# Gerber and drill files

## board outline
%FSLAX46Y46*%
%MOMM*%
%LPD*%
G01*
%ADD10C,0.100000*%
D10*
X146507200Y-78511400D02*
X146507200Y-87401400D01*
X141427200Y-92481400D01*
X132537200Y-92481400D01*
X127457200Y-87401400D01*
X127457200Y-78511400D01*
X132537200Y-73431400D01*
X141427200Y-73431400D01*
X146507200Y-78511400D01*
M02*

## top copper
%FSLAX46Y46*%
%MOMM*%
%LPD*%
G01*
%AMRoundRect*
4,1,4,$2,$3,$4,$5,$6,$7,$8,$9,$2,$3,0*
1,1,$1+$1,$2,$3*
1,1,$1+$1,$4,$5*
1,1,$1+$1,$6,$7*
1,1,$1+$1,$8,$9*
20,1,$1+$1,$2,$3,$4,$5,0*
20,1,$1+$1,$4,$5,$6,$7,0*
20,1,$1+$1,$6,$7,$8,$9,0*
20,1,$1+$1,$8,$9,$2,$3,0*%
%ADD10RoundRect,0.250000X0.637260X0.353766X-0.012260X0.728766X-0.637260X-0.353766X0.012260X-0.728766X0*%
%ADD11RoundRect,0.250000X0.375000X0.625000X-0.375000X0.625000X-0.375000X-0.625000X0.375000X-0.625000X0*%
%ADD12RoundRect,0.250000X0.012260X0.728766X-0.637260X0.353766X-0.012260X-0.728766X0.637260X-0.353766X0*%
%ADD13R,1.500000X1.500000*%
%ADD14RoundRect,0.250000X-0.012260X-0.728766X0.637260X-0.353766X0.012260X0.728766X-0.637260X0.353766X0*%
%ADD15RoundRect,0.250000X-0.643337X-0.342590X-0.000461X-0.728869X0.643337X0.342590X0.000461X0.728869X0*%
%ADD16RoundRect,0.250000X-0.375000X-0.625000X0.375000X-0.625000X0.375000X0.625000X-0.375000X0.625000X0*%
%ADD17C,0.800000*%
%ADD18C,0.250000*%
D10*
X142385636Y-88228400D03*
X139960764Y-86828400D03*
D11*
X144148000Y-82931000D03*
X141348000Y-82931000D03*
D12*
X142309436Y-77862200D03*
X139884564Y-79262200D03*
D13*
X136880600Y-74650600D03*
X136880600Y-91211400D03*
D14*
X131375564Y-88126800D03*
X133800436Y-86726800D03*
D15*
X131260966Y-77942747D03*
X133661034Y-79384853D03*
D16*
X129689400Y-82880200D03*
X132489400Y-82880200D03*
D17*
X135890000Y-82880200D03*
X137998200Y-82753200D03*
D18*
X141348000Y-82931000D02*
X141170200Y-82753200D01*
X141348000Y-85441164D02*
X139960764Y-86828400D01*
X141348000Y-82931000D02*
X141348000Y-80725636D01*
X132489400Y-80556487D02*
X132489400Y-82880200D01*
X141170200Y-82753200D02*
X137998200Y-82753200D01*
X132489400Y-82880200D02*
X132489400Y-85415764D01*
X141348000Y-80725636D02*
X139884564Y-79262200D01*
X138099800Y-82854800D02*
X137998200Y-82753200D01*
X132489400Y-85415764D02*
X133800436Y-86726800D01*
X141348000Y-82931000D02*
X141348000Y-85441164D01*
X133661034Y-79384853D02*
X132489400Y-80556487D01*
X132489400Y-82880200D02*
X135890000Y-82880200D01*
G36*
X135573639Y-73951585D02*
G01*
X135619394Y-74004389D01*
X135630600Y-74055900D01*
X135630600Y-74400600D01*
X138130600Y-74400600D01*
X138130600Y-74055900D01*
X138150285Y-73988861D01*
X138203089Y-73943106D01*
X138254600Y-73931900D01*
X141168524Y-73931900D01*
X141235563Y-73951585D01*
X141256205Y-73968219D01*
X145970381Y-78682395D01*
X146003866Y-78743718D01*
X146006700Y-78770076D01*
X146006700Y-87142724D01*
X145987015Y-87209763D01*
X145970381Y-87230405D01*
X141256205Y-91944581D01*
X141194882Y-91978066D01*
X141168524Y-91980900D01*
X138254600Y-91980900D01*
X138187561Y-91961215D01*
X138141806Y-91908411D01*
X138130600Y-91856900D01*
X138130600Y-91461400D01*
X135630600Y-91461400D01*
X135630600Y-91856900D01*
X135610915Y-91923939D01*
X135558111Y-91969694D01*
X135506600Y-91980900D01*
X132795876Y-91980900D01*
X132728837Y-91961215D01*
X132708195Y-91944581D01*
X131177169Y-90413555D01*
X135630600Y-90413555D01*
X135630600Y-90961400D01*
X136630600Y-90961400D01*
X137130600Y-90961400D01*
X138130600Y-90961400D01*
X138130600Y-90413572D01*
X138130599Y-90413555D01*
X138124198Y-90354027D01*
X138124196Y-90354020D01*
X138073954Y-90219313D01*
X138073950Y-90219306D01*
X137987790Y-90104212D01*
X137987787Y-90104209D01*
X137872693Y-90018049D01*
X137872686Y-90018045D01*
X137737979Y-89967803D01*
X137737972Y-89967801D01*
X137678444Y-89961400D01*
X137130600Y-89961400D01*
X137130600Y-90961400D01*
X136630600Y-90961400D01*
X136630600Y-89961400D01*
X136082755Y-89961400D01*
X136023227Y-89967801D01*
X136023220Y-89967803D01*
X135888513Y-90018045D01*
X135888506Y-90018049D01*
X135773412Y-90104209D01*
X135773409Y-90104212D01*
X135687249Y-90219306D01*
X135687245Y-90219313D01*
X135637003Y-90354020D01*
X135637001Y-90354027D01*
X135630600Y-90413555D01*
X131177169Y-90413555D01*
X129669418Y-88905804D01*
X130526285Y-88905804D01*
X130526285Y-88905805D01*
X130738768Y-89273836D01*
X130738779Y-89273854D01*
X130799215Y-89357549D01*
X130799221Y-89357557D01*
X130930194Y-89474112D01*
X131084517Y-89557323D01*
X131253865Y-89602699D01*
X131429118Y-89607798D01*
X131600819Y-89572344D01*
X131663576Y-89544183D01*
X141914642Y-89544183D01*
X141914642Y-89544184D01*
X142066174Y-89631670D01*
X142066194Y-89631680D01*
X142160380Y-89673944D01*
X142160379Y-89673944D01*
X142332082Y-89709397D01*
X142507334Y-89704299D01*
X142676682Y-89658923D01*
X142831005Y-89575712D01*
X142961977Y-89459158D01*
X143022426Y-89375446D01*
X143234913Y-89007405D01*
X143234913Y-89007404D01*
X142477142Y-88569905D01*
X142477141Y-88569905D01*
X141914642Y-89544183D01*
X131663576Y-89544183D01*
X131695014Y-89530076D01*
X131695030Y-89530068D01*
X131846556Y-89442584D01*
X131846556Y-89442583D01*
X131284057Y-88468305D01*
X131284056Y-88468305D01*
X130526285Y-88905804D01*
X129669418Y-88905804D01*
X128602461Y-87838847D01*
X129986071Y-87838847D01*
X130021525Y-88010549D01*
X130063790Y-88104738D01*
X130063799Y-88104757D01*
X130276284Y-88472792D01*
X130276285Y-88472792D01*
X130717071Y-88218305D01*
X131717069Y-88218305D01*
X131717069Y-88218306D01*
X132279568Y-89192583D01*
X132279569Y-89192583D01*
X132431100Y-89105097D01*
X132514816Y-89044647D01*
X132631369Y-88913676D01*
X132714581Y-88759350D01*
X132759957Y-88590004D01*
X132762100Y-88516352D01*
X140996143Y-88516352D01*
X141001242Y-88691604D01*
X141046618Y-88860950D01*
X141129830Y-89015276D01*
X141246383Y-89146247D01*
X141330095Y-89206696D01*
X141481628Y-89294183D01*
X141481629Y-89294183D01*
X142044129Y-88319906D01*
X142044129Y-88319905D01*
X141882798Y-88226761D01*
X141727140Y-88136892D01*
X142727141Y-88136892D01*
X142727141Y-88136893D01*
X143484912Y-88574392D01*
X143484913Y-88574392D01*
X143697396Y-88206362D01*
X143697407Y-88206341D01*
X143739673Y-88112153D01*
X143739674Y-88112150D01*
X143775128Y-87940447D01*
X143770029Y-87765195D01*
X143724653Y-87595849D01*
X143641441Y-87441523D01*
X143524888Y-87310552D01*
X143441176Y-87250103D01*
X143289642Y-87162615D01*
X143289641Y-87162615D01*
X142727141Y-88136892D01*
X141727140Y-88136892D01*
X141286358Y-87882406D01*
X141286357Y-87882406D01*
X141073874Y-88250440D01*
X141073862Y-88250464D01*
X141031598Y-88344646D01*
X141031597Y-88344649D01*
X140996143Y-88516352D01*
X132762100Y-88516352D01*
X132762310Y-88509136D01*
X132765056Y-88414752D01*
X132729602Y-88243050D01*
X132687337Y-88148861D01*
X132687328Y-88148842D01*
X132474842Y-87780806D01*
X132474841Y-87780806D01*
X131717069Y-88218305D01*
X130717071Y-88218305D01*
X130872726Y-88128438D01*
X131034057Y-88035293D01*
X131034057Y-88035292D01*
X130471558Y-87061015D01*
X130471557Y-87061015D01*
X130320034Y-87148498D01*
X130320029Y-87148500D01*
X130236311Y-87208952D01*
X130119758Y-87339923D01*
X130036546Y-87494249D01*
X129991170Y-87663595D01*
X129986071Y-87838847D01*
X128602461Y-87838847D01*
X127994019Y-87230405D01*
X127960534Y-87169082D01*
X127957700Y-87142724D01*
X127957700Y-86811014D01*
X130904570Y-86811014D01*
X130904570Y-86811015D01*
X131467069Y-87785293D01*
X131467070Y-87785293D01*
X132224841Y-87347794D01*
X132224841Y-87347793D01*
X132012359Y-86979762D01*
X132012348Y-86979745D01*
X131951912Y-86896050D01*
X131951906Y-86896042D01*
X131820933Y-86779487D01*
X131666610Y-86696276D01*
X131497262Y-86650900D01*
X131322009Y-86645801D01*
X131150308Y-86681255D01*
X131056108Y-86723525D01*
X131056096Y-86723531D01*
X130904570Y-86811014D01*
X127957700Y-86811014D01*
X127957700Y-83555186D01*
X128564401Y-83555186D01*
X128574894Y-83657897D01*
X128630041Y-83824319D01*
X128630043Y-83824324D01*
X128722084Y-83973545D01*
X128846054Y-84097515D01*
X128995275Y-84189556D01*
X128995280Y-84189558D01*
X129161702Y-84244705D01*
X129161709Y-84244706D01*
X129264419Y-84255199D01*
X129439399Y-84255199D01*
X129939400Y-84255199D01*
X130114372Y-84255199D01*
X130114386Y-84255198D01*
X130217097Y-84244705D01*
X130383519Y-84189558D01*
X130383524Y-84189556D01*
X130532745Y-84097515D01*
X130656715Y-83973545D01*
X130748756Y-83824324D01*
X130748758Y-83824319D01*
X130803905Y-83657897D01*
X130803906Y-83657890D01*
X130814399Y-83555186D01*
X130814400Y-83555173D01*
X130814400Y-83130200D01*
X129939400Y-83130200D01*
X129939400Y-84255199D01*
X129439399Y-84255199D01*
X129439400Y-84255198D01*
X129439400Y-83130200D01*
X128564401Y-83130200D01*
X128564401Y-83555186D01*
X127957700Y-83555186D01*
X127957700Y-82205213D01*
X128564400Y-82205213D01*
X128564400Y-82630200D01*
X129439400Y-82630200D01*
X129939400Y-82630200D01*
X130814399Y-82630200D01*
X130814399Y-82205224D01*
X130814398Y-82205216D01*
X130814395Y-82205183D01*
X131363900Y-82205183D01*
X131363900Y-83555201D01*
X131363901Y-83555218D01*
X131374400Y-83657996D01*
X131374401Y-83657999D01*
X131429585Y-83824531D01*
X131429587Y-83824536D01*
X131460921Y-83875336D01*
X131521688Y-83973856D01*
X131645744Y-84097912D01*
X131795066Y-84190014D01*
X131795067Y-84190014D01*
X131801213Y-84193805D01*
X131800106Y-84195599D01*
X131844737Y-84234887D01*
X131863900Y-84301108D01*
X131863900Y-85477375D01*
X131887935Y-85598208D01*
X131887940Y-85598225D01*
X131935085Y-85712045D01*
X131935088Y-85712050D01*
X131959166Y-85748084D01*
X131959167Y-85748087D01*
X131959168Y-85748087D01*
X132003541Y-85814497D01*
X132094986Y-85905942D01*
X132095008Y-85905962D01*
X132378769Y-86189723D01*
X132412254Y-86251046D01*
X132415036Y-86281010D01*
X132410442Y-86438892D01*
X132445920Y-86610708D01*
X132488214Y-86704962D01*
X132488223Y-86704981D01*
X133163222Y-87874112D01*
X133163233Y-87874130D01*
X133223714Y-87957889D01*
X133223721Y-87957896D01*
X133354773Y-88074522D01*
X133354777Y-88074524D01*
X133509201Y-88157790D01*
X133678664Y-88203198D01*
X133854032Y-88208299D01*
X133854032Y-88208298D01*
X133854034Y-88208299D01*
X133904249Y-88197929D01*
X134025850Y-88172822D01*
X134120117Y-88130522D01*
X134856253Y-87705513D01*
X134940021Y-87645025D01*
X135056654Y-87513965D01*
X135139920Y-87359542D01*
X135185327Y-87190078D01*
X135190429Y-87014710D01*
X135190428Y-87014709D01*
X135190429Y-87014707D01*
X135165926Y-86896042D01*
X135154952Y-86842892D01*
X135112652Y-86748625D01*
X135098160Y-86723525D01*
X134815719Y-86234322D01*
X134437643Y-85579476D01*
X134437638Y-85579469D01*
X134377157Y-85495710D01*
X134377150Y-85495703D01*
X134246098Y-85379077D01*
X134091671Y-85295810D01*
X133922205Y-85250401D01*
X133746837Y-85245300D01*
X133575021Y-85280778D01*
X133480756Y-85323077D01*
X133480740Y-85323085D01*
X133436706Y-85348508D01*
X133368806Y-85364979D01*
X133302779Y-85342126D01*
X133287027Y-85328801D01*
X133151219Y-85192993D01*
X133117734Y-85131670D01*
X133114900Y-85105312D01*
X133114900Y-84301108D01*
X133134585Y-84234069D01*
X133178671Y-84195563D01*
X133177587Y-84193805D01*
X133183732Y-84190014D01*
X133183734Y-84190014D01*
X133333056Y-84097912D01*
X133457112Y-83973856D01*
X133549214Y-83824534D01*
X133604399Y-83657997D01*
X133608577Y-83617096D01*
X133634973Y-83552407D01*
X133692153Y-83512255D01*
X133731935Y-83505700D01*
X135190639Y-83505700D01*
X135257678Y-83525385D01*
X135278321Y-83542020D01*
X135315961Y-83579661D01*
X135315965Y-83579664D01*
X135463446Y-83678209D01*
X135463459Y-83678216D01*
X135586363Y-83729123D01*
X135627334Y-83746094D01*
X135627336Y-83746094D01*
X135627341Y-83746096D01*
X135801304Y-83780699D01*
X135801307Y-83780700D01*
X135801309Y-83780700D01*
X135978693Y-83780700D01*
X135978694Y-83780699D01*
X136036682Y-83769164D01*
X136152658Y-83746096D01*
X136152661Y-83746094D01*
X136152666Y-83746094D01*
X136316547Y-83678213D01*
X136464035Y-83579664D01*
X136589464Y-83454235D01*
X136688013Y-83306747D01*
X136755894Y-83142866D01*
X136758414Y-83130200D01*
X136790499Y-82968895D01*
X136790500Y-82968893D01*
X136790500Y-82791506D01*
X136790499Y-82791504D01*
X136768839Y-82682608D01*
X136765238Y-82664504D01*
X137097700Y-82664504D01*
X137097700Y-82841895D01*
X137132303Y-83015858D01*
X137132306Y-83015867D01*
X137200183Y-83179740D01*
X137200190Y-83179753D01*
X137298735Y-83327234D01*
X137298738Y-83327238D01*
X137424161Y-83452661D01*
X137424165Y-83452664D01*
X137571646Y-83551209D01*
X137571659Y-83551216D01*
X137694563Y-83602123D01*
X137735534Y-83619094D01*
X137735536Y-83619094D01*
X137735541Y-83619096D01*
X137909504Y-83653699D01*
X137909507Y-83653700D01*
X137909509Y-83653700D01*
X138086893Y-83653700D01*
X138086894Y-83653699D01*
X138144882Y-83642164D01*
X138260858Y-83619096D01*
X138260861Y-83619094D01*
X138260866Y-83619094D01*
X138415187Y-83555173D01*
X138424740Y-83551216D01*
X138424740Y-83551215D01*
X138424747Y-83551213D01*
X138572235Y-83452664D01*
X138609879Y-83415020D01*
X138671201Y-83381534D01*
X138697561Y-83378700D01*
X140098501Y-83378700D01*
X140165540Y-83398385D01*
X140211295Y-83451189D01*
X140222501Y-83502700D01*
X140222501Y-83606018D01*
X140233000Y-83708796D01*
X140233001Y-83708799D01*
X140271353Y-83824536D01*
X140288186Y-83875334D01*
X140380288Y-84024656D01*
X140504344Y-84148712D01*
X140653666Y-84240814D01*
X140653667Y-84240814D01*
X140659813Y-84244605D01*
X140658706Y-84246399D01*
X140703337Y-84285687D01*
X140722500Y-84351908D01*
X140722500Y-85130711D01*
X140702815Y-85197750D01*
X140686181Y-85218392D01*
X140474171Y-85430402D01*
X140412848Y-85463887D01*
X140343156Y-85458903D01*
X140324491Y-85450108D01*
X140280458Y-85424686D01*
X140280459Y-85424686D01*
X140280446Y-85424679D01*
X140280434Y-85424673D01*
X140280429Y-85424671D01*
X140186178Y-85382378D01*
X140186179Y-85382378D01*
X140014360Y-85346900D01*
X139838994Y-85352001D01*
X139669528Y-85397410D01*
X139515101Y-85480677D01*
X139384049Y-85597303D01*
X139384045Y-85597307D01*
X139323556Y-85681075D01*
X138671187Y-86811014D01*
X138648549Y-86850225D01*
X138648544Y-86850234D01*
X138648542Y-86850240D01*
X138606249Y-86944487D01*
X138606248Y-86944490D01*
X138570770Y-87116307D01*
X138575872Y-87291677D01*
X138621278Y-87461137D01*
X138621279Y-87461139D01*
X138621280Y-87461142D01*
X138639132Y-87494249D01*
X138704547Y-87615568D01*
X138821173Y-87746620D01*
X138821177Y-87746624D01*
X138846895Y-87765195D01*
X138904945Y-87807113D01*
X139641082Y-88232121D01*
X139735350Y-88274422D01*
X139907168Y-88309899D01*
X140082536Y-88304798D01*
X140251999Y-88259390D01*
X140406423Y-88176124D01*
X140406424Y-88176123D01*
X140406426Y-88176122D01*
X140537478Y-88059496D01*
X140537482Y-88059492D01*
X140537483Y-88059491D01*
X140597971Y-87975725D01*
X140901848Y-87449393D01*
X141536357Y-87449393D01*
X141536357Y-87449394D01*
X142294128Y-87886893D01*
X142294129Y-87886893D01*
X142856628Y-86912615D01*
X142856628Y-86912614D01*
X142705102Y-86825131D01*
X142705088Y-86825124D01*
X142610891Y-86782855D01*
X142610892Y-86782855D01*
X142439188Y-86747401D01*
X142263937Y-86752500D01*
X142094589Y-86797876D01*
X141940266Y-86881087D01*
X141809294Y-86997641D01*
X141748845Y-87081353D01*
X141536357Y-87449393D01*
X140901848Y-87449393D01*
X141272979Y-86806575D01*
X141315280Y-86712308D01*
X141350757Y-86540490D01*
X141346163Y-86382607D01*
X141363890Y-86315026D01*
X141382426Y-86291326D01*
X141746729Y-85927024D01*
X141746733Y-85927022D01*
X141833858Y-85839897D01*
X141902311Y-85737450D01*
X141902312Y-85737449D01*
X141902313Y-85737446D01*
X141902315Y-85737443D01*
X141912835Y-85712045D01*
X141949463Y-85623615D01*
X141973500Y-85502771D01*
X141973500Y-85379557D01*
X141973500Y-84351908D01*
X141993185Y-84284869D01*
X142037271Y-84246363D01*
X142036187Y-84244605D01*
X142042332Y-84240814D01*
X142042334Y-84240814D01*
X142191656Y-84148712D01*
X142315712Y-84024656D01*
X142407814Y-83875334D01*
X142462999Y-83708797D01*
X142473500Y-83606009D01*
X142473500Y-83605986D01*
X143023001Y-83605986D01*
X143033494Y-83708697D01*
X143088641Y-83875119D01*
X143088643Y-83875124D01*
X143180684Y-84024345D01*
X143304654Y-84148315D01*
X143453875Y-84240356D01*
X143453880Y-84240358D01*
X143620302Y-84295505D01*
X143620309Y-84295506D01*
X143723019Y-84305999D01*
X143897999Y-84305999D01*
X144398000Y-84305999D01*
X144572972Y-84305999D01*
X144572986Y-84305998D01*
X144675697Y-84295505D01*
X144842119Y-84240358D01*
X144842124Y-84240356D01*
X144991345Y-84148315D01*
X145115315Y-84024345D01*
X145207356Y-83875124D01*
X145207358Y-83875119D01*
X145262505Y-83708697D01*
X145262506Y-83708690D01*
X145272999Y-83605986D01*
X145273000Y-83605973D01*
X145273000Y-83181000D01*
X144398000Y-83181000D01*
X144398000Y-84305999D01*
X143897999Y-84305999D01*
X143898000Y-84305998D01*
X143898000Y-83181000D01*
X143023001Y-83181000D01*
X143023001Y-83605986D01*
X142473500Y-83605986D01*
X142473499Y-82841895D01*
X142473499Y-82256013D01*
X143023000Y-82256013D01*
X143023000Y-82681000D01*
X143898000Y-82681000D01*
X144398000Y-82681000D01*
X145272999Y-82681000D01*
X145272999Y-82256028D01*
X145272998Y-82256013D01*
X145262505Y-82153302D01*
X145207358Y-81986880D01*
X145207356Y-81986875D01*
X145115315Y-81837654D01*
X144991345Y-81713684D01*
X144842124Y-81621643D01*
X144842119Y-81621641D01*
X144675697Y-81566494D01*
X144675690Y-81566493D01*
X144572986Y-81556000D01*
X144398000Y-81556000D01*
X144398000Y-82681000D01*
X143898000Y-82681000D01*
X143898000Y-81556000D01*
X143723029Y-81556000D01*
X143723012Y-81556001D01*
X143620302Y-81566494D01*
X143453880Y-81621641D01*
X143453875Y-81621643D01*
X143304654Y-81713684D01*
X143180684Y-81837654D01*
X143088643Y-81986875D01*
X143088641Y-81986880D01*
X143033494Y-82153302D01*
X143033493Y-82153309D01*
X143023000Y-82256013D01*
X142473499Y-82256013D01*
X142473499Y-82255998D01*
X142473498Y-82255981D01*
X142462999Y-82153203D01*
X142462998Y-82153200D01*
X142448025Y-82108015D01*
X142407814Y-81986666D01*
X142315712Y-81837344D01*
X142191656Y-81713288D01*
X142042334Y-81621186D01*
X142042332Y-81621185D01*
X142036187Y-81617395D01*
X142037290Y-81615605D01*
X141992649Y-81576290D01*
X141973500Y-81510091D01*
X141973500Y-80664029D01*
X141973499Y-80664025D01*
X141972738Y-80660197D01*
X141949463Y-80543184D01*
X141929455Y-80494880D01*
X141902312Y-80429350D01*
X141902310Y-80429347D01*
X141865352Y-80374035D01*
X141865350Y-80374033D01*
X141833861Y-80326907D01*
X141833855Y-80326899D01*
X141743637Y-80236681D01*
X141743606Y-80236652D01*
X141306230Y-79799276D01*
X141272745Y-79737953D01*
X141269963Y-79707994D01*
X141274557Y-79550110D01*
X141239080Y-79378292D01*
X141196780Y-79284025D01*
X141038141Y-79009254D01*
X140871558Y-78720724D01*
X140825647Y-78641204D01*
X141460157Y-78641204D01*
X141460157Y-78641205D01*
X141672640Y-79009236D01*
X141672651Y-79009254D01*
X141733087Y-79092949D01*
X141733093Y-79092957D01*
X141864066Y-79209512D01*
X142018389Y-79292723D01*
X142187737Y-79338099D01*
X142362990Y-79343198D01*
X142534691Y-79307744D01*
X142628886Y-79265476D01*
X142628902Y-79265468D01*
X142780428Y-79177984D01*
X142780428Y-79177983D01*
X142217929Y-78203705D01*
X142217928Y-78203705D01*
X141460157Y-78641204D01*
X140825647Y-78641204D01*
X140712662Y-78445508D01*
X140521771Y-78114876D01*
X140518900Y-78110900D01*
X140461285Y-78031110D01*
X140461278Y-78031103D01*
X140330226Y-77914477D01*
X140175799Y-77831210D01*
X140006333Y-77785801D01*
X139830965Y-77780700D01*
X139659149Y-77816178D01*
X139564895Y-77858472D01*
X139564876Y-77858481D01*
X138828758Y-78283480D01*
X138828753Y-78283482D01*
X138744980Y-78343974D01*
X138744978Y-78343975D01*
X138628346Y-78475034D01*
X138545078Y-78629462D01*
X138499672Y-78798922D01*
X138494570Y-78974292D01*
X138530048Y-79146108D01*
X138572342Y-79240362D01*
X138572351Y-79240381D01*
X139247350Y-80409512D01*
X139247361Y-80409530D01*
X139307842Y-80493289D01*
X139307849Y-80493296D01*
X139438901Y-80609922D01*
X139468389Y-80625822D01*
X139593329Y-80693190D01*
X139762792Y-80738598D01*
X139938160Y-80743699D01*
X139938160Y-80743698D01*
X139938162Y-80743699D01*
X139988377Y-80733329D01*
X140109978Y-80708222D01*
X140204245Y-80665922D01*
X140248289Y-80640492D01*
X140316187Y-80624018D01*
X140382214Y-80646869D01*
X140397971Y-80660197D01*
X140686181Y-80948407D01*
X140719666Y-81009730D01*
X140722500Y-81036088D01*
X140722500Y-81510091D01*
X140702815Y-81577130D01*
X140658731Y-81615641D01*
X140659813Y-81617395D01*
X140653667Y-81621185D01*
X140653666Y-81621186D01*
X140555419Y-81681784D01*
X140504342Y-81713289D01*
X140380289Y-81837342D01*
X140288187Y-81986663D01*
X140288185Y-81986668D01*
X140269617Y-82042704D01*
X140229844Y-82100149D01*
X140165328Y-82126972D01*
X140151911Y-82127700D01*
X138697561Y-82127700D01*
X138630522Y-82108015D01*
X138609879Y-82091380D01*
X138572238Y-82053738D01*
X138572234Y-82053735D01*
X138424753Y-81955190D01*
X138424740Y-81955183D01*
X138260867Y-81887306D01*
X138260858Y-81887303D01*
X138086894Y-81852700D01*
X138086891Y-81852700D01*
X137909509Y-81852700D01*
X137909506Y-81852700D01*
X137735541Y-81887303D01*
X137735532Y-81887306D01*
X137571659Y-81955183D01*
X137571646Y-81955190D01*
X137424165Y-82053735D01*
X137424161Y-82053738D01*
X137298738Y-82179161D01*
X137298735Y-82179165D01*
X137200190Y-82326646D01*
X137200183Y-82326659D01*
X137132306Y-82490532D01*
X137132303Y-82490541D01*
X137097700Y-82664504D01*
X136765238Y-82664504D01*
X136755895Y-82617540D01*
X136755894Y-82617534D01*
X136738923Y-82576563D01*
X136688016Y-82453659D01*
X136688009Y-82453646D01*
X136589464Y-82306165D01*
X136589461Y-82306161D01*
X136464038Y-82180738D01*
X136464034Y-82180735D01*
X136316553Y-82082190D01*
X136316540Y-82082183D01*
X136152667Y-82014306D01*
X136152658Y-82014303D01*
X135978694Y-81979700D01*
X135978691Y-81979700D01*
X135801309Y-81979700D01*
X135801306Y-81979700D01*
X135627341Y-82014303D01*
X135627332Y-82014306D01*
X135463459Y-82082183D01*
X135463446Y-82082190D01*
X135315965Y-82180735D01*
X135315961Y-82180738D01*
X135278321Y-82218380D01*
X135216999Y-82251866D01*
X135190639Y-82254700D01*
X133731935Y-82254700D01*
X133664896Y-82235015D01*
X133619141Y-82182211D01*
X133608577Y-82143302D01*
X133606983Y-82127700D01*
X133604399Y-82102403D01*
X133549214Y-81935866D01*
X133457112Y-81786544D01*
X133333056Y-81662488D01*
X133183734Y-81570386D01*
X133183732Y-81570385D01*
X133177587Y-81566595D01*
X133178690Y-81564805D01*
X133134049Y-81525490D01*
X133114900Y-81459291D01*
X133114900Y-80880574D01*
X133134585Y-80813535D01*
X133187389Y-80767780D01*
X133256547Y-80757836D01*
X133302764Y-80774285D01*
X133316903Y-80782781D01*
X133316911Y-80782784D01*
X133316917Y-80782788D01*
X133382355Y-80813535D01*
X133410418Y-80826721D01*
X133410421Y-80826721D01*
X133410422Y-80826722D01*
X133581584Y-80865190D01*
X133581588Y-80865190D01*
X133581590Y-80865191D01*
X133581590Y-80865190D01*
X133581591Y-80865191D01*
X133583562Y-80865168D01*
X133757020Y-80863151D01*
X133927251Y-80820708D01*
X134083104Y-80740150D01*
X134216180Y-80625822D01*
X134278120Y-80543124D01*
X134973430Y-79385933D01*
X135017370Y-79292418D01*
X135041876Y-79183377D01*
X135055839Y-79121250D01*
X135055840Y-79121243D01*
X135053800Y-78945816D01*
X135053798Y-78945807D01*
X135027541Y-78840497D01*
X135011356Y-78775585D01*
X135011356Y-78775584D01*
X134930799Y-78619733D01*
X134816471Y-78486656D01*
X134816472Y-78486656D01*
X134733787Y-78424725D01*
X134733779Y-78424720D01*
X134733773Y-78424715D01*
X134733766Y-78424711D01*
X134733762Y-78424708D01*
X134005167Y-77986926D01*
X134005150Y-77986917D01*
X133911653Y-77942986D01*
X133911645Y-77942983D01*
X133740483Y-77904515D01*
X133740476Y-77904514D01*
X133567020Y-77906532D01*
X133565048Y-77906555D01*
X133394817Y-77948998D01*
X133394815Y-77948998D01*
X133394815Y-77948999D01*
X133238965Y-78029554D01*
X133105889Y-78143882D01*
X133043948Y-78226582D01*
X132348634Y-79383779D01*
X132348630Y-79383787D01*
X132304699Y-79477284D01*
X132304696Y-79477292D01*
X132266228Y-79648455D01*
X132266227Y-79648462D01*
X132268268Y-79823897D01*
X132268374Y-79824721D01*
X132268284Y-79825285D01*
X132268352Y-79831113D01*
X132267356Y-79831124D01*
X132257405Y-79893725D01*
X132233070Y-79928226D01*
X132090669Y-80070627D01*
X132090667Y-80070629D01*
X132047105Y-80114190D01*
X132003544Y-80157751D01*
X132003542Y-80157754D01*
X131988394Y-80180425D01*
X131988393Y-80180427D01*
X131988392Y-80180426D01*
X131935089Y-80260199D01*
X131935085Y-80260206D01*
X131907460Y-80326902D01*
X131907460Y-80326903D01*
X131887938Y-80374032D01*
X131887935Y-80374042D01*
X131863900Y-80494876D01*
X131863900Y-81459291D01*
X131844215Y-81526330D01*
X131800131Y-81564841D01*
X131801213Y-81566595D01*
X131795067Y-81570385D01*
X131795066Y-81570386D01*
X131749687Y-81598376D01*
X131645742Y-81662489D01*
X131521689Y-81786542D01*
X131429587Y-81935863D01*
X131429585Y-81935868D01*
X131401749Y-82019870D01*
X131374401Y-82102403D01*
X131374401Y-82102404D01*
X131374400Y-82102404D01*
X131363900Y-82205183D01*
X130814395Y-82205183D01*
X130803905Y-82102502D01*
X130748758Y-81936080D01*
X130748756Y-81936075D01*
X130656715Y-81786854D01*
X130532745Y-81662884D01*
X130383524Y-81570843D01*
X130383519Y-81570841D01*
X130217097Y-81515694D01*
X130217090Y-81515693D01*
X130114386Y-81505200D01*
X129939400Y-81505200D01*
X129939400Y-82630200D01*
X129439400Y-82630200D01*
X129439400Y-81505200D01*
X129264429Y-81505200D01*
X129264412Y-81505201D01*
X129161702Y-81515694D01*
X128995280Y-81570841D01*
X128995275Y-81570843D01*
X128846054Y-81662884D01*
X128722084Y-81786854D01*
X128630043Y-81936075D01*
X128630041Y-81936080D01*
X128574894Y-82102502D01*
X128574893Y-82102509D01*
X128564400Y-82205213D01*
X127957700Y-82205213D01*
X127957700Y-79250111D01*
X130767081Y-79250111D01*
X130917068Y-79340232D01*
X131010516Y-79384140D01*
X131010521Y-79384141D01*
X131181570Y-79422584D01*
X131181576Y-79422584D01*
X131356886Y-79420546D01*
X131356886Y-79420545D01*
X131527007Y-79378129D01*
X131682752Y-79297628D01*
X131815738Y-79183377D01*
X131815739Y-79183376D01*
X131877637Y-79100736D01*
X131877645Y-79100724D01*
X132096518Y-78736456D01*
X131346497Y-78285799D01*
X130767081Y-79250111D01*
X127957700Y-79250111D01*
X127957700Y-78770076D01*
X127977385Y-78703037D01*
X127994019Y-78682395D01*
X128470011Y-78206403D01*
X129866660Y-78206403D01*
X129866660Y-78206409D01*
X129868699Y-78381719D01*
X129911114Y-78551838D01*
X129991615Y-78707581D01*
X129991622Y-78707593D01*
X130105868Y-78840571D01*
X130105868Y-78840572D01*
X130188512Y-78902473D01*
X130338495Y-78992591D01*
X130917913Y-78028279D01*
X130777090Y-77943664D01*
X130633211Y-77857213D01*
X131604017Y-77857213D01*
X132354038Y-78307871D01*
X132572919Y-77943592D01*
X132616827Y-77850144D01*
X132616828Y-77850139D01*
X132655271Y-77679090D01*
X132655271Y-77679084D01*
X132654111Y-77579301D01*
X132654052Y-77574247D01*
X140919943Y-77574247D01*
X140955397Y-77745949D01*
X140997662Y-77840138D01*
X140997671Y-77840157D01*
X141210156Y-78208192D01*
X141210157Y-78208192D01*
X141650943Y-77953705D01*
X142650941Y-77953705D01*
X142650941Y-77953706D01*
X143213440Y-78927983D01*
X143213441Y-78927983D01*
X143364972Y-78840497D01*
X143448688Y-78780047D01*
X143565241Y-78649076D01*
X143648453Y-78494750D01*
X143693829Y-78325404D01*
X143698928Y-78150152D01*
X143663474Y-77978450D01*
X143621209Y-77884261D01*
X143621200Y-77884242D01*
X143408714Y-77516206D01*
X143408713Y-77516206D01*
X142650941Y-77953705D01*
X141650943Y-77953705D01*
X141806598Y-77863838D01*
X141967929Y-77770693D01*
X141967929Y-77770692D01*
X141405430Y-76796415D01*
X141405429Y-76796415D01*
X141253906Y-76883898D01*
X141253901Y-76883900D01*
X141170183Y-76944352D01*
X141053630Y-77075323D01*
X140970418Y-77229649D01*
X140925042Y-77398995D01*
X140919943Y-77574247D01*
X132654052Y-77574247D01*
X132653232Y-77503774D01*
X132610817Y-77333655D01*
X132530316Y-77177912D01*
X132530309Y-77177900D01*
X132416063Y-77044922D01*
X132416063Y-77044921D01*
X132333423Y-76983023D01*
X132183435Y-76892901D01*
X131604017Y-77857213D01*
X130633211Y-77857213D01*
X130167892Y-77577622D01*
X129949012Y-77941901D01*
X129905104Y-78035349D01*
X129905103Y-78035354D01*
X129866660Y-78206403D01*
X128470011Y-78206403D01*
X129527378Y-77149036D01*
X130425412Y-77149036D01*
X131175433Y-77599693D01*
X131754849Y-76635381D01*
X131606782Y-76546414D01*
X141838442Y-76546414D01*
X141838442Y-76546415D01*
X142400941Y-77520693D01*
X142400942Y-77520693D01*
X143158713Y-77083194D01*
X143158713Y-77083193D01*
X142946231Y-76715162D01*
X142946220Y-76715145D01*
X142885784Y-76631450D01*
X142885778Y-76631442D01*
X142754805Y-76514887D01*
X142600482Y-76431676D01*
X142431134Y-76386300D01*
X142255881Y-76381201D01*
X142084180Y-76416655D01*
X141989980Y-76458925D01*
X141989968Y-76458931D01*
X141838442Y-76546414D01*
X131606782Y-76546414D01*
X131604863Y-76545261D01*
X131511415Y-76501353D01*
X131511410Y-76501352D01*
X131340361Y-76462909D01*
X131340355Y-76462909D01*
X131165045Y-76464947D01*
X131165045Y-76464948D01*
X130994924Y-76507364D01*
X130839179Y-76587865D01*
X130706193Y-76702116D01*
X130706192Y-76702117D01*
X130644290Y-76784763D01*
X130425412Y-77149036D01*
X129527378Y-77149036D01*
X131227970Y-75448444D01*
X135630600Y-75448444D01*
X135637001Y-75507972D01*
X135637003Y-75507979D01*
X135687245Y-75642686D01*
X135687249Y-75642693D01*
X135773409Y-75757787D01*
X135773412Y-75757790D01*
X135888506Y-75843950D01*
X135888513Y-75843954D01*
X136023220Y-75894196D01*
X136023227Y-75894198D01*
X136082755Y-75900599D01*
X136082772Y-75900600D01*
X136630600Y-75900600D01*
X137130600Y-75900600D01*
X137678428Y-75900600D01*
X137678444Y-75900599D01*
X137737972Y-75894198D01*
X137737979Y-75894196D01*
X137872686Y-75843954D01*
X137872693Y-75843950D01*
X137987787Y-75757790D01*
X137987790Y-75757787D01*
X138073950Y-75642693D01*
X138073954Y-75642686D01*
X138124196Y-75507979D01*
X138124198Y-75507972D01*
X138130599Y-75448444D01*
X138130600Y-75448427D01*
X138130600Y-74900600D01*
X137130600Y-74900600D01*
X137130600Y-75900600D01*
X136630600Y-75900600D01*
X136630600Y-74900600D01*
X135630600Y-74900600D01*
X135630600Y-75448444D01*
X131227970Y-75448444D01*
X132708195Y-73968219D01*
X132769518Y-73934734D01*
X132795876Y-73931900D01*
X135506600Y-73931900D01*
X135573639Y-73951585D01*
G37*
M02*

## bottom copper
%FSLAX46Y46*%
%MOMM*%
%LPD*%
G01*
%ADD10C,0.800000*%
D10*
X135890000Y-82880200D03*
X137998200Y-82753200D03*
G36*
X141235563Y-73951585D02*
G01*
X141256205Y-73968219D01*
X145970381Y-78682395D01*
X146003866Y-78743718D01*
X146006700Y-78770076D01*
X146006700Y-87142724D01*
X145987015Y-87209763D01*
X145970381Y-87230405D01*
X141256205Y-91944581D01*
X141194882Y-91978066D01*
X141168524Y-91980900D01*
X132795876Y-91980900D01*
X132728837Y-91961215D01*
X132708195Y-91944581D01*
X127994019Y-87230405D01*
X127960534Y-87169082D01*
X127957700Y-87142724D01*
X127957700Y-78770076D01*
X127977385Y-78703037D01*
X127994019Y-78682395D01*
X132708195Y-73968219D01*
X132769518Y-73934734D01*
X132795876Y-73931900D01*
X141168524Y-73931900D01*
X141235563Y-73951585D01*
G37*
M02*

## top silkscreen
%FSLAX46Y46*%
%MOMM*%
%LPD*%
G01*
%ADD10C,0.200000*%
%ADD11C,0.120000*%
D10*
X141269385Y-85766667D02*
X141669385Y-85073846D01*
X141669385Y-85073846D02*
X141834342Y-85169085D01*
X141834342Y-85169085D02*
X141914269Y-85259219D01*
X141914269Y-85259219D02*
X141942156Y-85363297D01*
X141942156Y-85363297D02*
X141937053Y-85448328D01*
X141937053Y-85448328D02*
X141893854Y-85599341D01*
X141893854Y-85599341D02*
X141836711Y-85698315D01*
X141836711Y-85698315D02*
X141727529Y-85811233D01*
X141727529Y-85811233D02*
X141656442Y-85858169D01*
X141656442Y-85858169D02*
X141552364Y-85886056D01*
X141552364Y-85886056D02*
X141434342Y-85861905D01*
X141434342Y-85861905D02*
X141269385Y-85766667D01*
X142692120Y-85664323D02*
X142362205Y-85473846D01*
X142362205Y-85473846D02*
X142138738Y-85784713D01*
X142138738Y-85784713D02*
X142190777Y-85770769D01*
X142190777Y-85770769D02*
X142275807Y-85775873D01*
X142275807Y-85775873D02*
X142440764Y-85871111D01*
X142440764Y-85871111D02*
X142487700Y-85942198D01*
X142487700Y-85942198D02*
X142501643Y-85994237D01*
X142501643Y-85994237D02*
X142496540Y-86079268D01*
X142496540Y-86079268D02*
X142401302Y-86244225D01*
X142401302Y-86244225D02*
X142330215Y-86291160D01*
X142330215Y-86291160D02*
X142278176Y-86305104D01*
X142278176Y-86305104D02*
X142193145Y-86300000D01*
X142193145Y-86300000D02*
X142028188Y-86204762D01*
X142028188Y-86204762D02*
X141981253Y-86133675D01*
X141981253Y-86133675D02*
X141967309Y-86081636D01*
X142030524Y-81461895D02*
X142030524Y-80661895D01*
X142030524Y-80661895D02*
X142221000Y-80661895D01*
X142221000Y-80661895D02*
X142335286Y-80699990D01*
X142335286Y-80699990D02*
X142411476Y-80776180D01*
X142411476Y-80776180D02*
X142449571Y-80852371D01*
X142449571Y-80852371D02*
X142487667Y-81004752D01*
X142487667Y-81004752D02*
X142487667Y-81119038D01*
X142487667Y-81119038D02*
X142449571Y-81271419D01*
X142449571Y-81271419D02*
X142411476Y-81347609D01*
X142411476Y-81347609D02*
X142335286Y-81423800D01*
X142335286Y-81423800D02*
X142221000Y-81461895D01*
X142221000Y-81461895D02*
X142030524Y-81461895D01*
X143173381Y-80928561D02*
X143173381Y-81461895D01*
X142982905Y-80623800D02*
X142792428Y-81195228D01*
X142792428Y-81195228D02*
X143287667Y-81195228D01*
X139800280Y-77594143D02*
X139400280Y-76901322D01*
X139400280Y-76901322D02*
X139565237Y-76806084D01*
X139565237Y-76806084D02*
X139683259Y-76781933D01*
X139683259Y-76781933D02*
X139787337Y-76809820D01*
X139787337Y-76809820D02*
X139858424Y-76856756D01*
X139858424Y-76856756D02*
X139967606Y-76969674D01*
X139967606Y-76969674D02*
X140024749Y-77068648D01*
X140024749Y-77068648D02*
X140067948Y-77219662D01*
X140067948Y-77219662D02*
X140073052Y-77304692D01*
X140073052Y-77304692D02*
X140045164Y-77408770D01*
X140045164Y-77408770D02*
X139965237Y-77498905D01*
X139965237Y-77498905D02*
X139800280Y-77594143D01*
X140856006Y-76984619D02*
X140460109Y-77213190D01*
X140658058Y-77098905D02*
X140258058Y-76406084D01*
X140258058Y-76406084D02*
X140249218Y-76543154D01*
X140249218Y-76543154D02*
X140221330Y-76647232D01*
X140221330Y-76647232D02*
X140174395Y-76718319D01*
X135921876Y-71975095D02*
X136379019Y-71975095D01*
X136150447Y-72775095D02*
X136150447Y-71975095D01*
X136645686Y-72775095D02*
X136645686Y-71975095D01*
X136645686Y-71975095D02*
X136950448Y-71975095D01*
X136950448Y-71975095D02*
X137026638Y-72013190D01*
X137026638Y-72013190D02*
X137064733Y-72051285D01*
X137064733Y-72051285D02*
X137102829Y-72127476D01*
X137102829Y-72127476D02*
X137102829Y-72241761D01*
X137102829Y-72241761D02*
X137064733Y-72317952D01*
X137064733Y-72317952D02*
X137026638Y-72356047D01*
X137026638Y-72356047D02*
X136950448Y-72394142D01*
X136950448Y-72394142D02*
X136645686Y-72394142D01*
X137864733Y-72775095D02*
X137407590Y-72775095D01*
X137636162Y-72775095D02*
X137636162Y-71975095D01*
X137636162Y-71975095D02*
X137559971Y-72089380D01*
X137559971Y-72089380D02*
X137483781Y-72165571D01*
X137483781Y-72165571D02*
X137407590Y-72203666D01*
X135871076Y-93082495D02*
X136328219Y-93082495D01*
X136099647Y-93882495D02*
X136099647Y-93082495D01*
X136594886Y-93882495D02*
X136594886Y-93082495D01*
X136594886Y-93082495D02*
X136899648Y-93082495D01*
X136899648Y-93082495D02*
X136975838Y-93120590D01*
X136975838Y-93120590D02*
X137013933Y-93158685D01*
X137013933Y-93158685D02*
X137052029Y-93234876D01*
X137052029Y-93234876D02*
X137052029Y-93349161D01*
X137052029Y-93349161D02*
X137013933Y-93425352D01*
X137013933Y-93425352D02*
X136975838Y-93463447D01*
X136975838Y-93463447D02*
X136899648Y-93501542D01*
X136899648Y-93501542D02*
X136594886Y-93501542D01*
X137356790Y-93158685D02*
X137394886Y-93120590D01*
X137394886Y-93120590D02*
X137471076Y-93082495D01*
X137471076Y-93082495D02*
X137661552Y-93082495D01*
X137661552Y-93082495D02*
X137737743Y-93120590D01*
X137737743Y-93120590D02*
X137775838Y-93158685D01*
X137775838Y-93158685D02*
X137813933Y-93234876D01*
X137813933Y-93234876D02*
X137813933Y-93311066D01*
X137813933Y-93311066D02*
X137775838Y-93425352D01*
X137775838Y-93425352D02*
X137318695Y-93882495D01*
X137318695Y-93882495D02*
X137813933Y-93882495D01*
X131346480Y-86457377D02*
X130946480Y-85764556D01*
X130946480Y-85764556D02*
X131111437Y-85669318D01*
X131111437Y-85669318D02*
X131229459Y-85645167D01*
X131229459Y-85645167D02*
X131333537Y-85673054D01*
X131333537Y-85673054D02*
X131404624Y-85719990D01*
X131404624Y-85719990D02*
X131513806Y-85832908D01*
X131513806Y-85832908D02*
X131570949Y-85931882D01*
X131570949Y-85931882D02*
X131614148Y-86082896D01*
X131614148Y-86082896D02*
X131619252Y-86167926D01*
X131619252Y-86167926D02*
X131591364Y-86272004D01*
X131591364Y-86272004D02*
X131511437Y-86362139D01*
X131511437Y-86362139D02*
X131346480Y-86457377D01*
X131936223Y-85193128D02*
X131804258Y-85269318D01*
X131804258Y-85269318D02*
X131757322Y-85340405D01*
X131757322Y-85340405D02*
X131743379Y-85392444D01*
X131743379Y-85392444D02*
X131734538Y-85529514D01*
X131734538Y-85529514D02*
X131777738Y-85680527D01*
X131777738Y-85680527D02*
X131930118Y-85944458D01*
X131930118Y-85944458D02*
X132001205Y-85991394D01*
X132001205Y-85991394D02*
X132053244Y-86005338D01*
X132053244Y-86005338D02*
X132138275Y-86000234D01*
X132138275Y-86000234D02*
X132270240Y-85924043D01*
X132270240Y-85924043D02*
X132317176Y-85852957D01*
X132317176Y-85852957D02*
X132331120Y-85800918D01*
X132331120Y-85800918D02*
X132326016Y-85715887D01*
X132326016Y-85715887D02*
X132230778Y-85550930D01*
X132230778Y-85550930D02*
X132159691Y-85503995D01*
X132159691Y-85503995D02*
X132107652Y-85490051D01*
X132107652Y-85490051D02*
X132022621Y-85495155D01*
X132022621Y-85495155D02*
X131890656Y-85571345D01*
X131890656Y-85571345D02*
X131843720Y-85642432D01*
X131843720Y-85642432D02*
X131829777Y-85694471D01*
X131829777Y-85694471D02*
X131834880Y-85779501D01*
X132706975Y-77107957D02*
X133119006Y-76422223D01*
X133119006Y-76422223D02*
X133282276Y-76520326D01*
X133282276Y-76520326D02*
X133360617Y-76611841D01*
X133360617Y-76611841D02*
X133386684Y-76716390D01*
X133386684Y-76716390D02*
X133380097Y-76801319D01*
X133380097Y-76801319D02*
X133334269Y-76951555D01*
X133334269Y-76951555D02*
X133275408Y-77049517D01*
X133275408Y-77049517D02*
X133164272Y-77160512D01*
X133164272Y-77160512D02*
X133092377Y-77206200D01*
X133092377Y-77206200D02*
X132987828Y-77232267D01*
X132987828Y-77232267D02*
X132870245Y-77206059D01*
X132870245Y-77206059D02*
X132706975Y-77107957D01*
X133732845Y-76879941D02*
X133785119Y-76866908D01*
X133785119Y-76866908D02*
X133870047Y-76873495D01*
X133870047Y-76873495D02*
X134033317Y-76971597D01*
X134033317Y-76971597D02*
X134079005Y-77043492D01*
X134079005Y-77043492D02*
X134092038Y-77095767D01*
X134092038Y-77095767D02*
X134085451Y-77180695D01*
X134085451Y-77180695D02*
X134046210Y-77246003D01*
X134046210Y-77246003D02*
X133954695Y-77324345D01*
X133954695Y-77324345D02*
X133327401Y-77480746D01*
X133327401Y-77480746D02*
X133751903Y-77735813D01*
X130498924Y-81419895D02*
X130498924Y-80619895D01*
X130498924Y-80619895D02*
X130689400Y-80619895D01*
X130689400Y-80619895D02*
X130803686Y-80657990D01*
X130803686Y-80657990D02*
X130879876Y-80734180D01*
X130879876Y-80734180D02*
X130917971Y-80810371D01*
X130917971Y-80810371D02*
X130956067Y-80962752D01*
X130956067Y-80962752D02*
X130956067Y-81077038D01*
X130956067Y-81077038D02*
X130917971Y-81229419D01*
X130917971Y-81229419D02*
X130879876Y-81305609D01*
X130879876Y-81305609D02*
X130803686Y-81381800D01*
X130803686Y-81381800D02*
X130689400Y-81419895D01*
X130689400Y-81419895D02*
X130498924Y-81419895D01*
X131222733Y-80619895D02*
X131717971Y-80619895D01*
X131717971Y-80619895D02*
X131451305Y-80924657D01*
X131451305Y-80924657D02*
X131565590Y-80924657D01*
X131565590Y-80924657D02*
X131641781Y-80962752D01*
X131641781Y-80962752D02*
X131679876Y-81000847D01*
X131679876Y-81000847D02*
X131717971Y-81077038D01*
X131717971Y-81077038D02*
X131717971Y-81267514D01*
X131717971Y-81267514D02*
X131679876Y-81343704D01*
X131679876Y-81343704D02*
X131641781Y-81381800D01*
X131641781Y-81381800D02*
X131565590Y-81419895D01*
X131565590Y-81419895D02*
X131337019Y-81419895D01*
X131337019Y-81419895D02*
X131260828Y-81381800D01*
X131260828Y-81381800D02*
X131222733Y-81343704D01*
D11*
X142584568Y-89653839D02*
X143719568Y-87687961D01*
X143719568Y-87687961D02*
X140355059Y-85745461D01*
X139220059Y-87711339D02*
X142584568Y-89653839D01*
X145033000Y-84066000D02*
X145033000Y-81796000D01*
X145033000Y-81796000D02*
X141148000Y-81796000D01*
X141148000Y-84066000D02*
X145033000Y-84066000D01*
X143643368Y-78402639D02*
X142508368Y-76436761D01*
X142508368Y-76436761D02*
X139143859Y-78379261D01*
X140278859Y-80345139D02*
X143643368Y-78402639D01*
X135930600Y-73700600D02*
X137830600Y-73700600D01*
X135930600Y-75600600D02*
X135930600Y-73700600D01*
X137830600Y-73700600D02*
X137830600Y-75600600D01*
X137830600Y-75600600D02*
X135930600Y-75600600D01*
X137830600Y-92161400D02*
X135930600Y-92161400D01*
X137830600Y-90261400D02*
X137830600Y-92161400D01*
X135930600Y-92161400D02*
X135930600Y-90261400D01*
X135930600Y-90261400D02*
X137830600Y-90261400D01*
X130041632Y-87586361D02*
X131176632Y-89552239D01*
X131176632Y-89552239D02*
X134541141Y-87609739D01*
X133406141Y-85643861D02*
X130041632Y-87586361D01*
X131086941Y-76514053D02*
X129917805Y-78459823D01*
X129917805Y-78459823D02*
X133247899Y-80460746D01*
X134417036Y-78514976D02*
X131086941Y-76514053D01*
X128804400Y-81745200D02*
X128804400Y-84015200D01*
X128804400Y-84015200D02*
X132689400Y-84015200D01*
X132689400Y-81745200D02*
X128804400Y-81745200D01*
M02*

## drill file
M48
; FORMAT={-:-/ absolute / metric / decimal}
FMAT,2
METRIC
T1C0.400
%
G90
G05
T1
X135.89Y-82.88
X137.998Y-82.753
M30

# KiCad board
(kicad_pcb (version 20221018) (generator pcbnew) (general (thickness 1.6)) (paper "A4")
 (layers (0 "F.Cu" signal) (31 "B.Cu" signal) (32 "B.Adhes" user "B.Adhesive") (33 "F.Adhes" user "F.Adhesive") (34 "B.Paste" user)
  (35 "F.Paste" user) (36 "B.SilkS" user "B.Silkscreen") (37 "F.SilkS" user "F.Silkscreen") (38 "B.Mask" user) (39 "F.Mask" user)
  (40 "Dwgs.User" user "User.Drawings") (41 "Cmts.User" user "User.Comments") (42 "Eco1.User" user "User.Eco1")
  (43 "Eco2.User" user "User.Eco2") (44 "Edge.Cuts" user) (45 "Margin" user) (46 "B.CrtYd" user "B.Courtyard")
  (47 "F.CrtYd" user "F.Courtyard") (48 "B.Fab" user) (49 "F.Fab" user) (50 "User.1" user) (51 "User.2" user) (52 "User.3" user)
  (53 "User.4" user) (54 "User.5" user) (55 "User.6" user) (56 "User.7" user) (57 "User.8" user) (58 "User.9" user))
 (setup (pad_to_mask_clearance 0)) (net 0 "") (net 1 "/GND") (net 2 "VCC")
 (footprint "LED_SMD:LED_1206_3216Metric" (layer "F.Cu") (at 141.1732 87.5284 150)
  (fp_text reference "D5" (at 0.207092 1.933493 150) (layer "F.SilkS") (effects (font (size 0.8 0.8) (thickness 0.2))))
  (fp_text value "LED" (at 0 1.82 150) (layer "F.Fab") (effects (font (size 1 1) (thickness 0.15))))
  (fp_line (start -2.285 -1.135) (end -2.285 1.135) (stroke (width 0.12) (type solid)) (layer "F.SilkS"))
  (fp_line (start -2.285 1.135) (end 1.6 1.135) (stroke (width 0.12) (type solid)) (layer "F.SilkS"))
  (fp_line (start 1.6 -1.135) (end -2.285 -1.135) (stroke (width 0.12) (type solid)) (layer "F.SilkS"))
  (pad "1" smd roundrect (at -1.4 0 150) (size 1.25 1.75) (layers "F.Cu" "F.Paste" "F.Mask") (roundrect_rratio 0.2) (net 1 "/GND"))
  (pad "2" smd roundrect (at 1.4 0 150) (size 1.25 1.75) (layers "F.Cu" "F.Paste" "F.Mask") (roundrect_rratio 0.2) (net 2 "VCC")))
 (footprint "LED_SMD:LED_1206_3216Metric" (layer "F.Cu") (at 142.748 82.931 180)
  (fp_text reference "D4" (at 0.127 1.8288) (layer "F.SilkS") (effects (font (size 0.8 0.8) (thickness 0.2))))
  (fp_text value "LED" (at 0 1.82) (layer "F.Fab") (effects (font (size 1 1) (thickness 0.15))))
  (fp_line (start -2.285 -1.135) (end -2.285 1.135) (stroke (width 0.12) (type solid)) (layer "F.SilkS"))
  (fp_line (start -2.285 1.135) (end 1.6 1.135) (stroke (width 0.12) (type solid)) (layer "F.SilkS"))
  (fp_line (start 1.6 -1.135) (end -2.285 -1.135) (stroke (width 0.12) (type solid)) (layer "F.SilkS"))
  (pad "1" smd roundrect (at -1.4 0 180) (size 1.25 1.75) (layers "F.Cu" "F.Paste" "F.Mask") (roundrect_rratio 0.2) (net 1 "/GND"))
  (pad "2" smd roundrect (at 1.4 0 180) (size 1.25 1.75) (layers "F.Cu" "F.Paste" "F.Mask") (roundrect_rratio 0.2) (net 2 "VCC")))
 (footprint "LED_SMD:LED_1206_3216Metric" (layer "F.Cu") (at 141.097 78.5622 -150)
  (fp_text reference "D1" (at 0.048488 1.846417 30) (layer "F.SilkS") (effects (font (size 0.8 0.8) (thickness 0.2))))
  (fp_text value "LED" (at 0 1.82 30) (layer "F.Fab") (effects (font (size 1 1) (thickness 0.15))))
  (fp_line (start -2.285 -1.135) (end -2.285 1.135) (stroke (width 0.12) (type solid)) (layer "F.SilkS"))
  (fp_line (start -2.285 1.135) (end 1.6 1.135) (stroke (width 0.12) (type solid)) (layer "F.SilkS"))
  (fp_line (start 1.6 -1.135) (end -2.285 -1.135) (stroke (width 0.12) (type solid)) (layer "F.SilkS"))
  (pad "1" smd roundrect (at -1.4 0 210) (size 1.25 1.75) (layers "F.Cu" "F.Paste" "F.Mask") (roundrect_rratio 0.2) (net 1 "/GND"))
  (pad "2" smd roundrect (at 1.4 0 210) (size 1.25 1.75) (layers "F.Cu" "F.Paste" "F.Mask") (roundrect_rratio 0.2) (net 2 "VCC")))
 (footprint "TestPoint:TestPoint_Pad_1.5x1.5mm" (layer "F.Cu") (at 136.8806 74.6506)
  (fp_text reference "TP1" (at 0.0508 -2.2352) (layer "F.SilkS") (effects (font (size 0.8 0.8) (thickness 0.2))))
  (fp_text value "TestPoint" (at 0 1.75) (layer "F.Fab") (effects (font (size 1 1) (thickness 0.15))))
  (fp_line (start -0.95 -0.95) (end 0.95 -0.95) (stroke (width 0.12) (type solid)) (layer "F.SilkS"))
  (fp_line (start -0.95 0.95) (end -0.95 -0.95) (stroke (width 0.12) (type solid)) (layer "F.SilkS"))
  (fp_line (start 0.95 -0.95) (end 0.95 0.95) (stroke (width 0.12) (type solid)) (layer "F.SilkS"))
  (fp_line (start 0.95 0.95) (end -0.95 0.95) (stroke (width 0.12) (type solid)) (layer "F.SilkS"))
  (pad "1" smd rect (at 0 0) (size 1.5 1.5) (layers "F.Cu" "F.Mask") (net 1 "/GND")))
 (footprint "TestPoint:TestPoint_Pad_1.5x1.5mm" (layer "F.Cu") (at 136.8806 91.2114 180)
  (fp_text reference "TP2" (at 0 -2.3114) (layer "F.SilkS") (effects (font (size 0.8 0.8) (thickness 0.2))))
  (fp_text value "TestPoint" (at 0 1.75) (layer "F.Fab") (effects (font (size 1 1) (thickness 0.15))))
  (fp_line (start -0.95 -0.95) (end 0.95 -0.95) (stroke (width 0.12) (type solid)) (layer "F.SilkS"))
  (fp_line (start -0.95 0.95) (end -0.95 -0.95) (stroke (width 0.12) (type solid)) (layer "F.SilkS"))
  (fp_line (start 0.95 -0.95) (end 0.95 0.95) (stroke (width 0.12) (type solid)) (layer "F.SilkS"))
  (fp_line (start 0.95 0.95) (end -0.95 0.95) (stroke (width 0.12) (type solid)) (layer "F.SilkS"))
  (pad "1" smd rect (at 0 0 180) (size 1.5 1.5) (layers "F.Cu" "F.Mask") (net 1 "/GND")))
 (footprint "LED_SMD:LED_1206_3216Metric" (layer "F.Cu") (at 132.588 87.4268 30)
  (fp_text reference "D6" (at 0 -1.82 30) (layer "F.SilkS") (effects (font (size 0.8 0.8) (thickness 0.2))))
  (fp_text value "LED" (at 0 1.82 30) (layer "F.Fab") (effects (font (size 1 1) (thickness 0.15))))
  (fp_line (start -2.285 -1.135) (end -2.285 1.135) (stroke (width 0.12) (type solid)) (layer "F.SilkS"))
  (fp_line (start -2.285 1.135) (end 1.6 1.135) (stroke (width 0.12) (type solid)) (layer "F.SilkS"))
  (fp_line (start 1.6 -1.135) (end -2.285 -1.135) (stroke (width 0.12) (type solid)) (layer "F.SilkS"))
  (pad "1" smd roundrect (at -1.4 0 30) (size 1.25 1.75) (layers "F.Cu" "F.Paste" "F.Mask") (roundrect_rratio 0.2) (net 1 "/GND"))
  (pad "2" smd roundrect (at 1.4 0 30) (size 1.25 1.75) (layers "F.Cu" "F.Paste" "F.Mask") (roundrect_rratio 0.2) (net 2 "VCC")))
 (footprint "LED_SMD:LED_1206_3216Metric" (layer "F.Cu") (at 132.461 78.6638 -31)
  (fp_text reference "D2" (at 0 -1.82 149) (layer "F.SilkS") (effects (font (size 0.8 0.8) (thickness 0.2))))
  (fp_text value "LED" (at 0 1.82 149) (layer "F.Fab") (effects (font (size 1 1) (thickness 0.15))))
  (fp_line (start -2.285 -1.135) (end -2.285 1.135) (stroke (width 0.12) (type solid)) (layer "F.SilkS"))
  (fp_line (start -2.285 1.135) (end 1.6 1.135) (stroke (width 0.12) (type solid)) (layer "F.SilkS"))
  (fp_line (start 1.6 -1.135) (end -2.285 -1.135) (stroke (width 0.12) (type solid)) (layer "F.SilkS"))
  (pad "1" smd roundrect (at -1.4 0 329) (size 1.25 1.75) (layers "F.Cu" "F.Paste" "F.Mask") (roundrect_rratio 0.2) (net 1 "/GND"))
  (pad "2" smd roundrect (at 1.4 0 329) (size 1.25 1.75) (layers "F.Cu" "F.Paste" "F.Mask") (roundrect_rratio 0.2) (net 2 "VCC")))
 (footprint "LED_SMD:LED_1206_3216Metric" (layer "F.Cu") (at 131.0894 82.8802)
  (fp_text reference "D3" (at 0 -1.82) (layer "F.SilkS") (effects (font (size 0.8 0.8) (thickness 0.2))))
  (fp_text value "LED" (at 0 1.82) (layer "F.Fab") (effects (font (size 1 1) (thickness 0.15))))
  (fp_line (start -2.285 -1.135) (end -2.285 1.135) (stroke (width 0.12) (type solid)) (layer "F.SilkS"))
  (fp_line (start -2.285 1.135) (end 1.6 1.135) (stroke (width 0.12) (type solid)) (layer "F.SilkS"))
  (fp_line (start 1.6 -1.135) (end -2.285 -1.135) (stroke (width 0.12) (type solid)) (layer "F.SilkS"))
  (pad "1" smd roundrect (at -1.4 0) (size 1.25 1.75) (layers "F.Cu" "F.Paste" "F.Mask") (roundrect_rratio 0.2) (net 1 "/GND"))
  (pad "2" smd roundrect (at 1.4 0) (size 1.25 1.75) (layers "F.Cu" "F.Paste" "F.Mask") (roundrect_rratio 0.2) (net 2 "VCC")))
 (gr_poly
  (pts (xy 146.5072 78.5114) (xy 146.5072 87.4014) (xy 141.4272 92.4814) (xy 132.5372 92.4814) (xy 127.4572 87.4014) (xy 127.4572 78.5114)
   (xy 132.5372 73.4314) (xy 141.4272 73.4314))
  (stroke (width 0.1) (type solid)) (fill none) (layer "Edge.Cuts"))
 (segment (start 141.348 82.931) (end 141.1702 82.7532) (width 0.25) (layer "F.Cu") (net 2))
 (segment (start 141.348 85.441164) (end 139.960764 86.8284) (width 0.25) (layer "F.Cu") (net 2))
 (segment (start 141.348 82.931) (end 141.348 80.725636) (width 0.25) (layer "F.Cu") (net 2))
 (segment (start 132.4894 80.556487) (end 132.4894 82.8802) (width 0.25) (layer "F.Cu") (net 2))
 (segment (start 141.1702 82.7532) (end 137.9982 82.7532) (width 0.25) (layer "F.Cu") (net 2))
 (segment (start 132.4894 82.8802) (end 132.4894 85.415764) (width 0.25) (layer "F.Cu") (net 2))
 (segment (start 141.348 80.725636) (end 139.884564 79.2622) (width 0.25) (layer "F.Cu") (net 2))
 (segment (start 138.0998 82.8548) (end 137.9982 82.7532) (width 0.25) (layer "F.Cu") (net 2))
 (segment (start 132.4894 85.415764) (end 133.800436 86.7268) (width 0.25) (layer "F.Cu") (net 2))
 (segment (start 141.348 82.931) (end 141.348 85.441164) (width 0.25) (layer "F.Cu") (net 2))
 (segment (start 133.661034 79.384853) (end 132.4894 80.556487) (width 0.25) (layer "F.Cu") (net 2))
 (segment (start 132.4894 82.8802) (end 135.89 82.8802) (width 0.25) (layer "F.Cu") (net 2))
 (via (at 135.89 82.8802) (size 0.8) (drill 0.4) (layers "F.Cu" "B.Cu") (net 2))
 (via (at 137.9982 82.7532) (size 0.8) (drill 0.4) (layers "F.Cu" "B.Cu") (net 2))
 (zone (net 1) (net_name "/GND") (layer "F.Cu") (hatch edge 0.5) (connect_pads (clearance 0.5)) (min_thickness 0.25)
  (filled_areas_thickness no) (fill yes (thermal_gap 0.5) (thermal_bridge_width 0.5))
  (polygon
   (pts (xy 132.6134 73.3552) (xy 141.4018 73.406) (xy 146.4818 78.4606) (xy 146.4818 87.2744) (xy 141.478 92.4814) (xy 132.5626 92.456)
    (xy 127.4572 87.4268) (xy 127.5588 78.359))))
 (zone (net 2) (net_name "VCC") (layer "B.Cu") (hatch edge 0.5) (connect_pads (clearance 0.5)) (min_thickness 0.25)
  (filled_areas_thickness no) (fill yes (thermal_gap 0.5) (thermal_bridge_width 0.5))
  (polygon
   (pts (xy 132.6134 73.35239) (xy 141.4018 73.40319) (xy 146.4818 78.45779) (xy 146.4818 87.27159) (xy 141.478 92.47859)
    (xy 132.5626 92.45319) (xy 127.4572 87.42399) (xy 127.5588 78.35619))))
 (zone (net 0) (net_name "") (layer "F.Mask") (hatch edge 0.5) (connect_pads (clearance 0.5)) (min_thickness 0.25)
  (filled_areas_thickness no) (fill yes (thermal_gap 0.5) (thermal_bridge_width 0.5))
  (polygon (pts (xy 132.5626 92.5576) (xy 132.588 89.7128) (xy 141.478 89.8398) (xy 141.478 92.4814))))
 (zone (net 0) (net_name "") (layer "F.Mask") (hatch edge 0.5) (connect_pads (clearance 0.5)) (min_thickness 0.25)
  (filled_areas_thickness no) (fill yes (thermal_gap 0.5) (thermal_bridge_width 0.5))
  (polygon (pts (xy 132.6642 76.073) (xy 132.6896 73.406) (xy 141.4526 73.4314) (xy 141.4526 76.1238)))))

